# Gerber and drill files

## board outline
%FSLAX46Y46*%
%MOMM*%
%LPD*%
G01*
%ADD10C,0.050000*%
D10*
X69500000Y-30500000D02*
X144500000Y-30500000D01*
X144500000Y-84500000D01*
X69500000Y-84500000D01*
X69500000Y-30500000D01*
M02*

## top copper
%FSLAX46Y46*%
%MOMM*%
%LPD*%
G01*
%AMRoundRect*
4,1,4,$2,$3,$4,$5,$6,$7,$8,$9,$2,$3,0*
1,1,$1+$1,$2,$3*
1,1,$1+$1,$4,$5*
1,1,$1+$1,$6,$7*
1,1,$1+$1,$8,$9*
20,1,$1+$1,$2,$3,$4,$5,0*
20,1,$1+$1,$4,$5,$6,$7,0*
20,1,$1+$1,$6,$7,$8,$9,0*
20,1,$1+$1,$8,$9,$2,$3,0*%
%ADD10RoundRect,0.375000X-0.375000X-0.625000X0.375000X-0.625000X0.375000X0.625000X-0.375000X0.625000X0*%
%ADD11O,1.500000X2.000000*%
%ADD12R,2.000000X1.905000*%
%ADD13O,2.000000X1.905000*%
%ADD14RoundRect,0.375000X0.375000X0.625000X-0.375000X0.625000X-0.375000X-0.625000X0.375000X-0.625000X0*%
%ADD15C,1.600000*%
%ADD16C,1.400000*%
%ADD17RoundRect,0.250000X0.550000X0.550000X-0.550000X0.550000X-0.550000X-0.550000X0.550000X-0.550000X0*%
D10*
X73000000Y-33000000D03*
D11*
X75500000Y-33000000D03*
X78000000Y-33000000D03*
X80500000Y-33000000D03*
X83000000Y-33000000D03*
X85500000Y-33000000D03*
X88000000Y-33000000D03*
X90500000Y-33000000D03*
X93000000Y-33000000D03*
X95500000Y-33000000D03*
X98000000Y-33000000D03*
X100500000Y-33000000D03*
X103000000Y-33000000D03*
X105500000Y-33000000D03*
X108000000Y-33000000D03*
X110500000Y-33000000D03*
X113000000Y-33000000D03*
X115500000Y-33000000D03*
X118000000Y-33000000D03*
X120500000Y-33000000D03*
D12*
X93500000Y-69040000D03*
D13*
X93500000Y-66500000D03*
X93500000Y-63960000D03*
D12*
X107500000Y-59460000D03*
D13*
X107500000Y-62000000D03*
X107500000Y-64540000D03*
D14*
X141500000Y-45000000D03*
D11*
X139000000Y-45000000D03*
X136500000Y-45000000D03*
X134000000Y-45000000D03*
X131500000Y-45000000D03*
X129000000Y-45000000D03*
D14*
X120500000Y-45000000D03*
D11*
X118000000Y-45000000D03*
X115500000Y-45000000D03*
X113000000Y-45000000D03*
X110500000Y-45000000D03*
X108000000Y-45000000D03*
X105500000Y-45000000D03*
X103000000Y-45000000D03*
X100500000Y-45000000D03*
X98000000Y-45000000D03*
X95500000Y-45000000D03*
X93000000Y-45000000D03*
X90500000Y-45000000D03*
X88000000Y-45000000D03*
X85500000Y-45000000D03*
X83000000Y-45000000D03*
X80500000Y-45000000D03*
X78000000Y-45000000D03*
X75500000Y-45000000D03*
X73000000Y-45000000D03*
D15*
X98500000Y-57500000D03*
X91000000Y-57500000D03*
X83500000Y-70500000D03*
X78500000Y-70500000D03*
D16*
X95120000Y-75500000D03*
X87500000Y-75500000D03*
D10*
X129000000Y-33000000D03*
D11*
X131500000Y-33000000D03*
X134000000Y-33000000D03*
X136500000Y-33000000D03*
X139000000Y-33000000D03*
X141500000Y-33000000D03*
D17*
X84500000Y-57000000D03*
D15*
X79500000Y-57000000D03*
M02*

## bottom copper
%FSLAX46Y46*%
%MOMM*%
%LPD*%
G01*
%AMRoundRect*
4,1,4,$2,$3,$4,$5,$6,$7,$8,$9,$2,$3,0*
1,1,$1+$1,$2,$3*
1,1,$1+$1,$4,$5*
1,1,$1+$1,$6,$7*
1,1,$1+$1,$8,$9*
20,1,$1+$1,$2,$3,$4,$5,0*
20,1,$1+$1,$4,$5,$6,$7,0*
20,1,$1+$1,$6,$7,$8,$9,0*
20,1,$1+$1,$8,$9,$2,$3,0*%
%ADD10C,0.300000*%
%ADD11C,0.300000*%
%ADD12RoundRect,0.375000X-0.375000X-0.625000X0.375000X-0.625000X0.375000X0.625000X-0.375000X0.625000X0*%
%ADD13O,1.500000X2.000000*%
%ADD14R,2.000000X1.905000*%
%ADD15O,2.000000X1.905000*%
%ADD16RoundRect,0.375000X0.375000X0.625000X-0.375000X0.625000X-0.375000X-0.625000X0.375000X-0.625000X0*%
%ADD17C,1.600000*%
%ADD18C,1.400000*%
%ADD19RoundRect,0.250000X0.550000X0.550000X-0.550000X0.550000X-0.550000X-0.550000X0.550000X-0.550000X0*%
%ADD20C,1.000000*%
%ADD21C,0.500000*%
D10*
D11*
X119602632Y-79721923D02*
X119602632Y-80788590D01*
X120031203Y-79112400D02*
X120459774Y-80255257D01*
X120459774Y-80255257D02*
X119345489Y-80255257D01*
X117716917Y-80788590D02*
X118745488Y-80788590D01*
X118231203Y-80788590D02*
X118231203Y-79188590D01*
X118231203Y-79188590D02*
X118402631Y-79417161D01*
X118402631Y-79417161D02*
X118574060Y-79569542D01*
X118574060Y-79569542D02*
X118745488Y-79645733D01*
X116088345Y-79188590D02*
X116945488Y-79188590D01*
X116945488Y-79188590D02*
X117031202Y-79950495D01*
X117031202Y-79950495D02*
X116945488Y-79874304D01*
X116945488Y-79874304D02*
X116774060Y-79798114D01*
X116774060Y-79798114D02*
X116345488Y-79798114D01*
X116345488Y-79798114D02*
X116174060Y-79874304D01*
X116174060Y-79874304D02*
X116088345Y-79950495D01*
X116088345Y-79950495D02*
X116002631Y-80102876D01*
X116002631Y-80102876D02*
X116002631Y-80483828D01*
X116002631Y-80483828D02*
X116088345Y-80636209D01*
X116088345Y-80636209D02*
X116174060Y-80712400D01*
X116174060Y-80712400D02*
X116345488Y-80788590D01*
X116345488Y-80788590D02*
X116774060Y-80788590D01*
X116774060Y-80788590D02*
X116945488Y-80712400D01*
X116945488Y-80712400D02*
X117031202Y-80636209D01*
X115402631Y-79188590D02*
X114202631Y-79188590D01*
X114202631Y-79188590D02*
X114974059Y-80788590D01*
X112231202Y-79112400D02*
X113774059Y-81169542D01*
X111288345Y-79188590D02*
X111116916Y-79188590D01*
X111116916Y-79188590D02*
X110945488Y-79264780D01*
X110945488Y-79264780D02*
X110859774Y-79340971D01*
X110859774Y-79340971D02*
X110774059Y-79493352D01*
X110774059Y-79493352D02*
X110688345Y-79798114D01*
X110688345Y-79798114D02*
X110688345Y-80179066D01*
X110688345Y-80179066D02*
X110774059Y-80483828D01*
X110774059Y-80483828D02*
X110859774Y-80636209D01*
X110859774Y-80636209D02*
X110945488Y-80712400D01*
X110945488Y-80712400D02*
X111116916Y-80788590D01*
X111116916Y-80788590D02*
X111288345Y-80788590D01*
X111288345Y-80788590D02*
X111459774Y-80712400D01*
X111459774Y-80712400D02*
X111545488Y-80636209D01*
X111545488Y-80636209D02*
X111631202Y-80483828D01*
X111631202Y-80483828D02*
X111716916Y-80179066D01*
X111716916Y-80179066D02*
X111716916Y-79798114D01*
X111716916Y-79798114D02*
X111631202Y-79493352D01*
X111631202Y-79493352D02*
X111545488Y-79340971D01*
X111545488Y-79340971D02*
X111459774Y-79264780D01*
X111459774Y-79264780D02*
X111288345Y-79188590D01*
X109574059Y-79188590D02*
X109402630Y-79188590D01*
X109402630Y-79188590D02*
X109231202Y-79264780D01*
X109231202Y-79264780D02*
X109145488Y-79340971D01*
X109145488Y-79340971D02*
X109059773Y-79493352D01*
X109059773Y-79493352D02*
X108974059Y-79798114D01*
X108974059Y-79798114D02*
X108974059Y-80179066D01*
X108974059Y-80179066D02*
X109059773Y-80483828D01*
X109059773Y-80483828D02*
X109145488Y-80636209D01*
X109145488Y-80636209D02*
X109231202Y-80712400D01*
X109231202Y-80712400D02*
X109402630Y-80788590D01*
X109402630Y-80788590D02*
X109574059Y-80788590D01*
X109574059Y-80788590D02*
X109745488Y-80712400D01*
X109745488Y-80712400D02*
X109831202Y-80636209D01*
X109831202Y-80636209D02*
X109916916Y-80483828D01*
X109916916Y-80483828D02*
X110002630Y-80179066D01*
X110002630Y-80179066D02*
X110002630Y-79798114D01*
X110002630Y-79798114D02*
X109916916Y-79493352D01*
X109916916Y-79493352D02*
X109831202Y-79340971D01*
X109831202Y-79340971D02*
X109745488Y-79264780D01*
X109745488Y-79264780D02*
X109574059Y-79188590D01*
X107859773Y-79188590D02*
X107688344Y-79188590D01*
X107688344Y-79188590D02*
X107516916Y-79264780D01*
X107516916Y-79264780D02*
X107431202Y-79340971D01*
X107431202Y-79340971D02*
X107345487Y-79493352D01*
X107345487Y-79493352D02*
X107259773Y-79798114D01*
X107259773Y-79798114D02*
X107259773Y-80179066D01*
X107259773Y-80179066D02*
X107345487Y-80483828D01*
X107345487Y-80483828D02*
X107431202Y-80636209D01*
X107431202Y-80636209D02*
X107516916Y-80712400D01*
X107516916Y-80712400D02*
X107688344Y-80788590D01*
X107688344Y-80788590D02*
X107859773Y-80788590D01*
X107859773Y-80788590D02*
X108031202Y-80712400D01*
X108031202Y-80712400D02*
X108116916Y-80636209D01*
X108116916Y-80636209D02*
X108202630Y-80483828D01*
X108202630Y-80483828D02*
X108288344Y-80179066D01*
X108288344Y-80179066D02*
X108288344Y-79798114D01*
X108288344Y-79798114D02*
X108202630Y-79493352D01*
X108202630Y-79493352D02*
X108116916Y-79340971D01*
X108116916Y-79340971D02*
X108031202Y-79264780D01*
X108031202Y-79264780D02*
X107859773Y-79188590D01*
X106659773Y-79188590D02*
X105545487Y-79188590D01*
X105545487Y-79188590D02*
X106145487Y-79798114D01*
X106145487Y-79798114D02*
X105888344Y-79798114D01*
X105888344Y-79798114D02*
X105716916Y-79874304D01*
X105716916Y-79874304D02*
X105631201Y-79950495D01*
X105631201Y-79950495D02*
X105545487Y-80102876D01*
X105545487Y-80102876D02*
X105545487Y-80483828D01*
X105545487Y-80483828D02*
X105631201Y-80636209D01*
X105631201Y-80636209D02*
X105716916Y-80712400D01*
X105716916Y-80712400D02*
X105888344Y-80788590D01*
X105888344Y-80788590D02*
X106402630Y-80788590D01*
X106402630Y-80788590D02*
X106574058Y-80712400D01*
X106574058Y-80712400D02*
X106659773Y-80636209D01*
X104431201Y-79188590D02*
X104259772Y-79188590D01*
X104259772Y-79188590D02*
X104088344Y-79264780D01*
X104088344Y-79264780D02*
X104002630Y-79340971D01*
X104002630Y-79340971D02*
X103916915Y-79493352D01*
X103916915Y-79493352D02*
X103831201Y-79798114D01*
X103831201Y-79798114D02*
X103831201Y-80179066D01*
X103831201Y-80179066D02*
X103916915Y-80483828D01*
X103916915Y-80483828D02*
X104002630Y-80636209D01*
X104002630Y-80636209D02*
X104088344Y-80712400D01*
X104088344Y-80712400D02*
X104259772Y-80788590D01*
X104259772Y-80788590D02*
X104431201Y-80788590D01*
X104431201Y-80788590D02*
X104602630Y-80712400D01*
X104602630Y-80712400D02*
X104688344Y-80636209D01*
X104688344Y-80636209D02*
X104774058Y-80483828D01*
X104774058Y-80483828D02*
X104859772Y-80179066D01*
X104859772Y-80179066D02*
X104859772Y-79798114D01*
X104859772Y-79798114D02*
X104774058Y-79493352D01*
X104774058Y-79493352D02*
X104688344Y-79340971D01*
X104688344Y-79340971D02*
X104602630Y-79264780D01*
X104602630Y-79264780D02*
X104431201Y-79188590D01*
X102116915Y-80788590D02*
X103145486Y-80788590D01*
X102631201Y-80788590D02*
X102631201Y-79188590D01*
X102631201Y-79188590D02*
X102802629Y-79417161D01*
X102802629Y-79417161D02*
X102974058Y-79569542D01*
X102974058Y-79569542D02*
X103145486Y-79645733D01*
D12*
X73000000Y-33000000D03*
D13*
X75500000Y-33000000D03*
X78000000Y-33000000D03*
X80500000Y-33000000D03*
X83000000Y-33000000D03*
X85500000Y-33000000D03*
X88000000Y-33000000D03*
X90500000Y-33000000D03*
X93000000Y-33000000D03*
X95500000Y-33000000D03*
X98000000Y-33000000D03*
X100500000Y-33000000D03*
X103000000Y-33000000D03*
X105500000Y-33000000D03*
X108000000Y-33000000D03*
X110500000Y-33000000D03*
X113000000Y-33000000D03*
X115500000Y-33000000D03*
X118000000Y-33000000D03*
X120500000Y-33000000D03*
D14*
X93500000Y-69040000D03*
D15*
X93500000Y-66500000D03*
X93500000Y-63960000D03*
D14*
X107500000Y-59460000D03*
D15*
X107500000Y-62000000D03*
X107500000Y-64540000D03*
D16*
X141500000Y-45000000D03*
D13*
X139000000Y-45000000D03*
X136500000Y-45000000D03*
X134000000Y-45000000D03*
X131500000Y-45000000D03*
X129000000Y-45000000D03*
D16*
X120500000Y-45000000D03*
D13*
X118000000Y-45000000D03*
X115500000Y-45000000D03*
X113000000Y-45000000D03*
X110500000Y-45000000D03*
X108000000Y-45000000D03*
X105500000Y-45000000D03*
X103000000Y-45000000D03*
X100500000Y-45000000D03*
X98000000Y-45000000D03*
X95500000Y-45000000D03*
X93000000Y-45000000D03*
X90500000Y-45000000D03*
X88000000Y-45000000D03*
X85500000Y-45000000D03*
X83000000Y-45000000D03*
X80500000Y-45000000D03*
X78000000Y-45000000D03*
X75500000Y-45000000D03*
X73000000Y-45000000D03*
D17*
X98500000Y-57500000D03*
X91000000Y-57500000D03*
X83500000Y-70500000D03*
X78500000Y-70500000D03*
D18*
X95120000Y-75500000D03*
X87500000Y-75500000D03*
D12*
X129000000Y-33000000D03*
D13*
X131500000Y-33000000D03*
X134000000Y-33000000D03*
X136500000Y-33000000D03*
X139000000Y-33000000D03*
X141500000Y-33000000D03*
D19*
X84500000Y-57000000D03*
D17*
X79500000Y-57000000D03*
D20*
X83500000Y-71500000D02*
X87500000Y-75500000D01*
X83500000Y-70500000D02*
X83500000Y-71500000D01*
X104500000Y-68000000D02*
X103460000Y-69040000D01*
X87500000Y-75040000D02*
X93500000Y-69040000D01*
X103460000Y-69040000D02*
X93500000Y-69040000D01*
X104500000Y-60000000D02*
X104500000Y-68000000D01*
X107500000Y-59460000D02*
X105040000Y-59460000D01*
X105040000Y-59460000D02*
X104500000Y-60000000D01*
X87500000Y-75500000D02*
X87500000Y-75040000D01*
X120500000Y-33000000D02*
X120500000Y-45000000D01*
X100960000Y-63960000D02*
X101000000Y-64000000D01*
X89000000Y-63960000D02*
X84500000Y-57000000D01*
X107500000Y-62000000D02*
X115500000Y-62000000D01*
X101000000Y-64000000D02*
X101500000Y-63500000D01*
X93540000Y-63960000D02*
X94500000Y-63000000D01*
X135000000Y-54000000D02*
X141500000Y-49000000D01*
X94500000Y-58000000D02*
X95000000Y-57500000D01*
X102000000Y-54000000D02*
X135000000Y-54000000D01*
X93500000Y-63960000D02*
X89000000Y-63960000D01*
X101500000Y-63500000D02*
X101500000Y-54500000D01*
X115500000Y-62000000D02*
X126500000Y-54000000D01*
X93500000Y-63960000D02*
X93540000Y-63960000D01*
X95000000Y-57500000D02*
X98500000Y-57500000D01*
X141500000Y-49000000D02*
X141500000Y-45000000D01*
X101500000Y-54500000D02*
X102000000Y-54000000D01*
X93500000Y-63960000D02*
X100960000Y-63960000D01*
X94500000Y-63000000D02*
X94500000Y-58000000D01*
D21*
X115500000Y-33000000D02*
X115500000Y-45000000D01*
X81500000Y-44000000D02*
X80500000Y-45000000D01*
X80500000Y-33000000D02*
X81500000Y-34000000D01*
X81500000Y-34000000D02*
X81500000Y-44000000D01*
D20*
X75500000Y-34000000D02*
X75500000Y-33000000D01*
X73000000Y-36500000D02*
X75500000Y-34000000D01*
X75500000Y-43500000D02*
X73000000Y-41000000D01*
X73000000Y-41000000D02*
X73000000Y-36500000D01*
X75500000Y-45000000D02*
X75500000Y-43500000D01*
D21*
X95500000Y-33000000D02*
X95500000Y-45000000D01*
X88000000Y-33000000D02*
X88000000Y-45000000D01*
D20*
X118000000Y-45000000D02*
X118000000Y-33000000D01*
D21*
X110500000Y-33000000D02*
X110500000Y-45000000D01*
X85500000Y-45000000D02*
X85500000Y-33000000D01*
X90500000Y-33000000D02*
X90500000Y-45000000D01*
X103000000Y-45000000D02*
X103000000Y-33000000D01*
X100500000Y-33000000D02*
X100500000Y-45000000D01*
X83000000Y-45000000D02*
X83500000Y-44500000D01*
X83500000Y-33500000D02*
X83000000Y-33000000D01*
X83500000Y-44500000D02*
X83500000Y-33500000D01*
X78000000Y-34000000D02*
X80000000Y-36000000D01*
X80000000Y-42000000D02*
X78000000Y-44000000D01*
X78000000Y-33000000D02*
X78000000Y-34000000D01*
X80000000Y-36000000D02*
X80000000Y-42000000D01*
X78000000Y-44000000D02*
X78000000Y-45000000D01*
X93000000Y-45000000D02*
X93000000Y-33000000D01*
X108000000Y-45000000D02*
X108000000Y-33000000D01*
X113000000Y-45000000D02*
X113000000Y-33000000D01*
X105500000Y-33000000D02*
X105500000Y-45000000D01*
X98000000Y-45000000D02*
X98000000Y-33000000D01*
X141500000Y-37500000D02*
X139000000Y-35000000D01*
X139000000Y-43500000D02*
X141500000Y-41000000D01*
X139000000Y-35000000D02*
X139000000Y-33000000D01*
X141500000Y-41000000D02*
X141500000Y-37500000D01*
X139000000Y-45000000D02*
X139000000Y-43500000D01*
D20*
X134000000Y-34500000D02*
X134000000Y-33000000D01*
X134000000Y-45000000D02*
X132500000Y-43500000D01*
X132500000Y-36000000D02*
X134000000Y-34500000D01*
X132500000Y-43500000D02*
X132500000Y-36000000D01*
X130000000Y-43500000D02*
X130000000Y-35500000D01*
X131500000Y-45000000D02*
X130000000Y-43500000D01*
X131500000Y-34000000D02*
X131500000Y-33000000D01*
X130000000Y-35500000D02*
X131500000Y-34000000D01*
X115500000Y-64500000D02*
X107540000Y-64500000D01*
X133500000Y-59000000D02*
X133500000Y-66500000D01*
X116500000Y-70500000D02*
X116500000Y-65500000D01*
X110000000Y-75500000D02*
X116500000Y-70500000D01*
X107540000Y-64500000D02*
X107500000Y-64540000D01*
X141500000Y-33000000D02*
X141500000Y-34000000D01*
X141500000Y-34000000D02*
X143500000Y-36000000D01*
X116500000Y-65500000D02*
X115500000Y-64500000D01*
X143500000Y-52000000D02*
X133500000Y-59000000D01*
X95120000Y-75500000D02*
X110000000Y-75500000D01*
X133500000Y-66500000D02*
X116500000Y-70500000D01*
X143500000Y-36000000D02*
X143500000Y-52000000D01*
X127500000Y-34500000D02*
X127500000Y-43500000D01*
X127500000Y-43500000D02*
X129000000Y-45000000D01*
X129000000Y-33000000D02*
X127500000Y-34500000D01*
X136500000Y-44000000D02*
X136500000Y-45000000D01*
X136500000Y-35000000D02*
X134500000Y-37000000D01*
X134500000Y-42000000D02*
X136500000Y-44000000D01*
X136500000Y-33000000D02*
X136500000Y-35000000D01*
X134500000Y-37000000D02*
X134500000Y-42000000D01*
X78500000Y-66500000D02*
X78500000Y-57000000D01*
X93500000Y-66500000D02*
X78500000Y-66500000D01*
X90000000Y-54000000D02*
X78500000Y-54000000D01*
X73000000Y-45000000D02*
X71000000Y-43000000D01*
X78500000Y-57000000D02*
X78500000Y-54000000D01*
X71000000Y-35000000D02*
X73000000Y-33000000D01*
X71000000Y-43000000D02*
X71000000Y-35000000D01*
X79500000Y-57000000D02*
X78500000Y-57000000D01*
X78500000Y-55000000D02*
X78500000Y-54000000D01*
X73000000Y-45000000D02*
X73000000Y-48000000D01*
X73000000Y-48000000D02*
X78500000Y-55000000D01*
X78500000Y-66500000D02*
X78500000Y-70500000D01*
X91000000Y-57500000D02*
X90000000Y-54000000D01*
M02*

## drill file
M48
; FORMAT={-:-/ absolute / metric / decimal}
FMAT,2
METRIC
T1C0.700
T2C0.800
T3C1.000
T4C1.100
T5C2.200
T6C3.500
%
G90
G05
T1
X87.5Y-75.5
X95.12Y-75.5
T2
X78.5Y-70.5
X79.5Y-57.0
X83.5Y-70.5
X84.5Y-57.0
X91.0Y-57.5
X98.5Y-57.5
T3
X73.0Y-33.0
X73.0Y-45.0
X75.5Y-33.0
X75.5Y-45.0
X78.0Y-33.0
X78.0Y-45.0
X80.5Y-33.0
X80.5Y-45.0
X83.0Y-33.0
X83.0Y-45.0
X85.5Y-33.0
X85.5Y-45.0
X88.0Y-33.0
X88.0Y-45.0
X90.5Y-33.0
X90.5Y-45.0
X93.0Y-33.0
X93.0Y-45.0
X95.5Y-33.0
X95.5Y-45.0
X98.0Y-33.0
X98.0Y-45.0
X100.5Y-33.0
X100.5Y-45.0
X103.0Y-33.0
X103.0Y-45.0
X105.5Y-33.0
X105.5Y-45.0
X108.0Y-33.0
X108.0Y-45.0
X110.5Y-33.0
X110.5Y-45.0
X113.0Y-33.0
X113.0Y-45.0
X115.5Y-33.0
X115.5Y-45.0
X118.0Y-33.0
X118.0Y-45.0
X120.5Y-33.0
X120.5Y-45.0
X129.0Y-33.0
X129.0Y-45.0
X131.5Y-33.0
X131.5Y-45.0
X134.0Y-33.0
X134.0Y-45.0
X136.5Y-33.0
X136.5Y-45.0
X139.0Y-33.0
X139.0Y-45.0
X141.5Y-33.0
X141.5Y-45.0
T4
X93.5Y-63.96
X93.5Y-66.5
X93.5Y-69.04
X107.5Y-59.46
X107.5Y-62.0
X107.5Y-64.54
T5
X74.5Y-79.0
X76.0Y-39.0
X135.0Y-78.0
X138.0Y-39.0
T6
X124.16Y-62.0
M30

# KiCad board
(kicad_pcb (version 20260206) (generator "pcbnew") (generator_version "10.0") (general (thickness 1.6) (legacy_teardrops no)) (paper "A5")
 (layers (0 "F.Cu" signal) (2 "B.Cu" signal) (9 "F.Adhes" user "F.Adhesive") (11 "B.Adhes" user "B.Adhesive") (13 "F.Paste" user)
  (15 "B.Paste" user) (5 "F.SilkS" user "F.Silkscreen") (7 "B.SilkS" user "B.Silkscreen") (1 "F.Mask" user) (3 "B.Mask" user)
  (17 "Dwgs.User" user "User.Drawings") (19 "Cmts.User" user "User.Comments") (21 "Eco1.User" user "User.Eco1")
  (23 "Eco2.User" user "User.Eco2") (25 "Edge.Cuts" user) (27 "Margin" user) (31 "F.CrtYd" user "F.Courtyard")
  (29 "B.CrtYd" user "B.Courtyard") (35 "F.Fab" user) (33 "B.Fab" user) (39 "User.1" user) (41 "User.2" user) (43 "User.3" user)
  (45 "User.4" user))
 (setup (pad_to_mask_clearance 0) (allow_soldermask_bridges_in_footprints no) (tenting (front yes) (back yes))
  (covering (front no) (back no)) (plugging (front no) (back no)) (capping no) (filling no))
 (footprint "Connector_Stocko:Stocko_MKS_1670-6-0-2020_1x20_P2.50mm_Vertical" (layer "F.Cu") (at 73 33)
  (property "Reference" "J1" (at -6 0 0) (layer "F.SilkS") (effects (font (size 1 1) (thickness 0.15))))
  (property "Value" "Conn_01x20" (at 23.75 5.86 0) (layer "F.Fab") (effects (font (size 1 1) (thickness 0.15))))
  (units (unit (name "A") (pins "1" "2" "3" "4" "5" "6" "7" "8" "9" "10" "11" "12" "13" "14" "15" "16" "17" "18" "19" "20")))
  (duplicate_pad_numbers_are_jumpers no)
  (pad "1" thru_hole roundrect (at 0 0) (size 1.5 2) (drill 1) (layers "*.Cu" "*.Mask") (remove_unused_layers no) (roundrect_rratio 0.25)
   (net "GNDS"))
  (pad "2" thru_hole oval (at 2.5 0) (size 1.5 2) (drill 1) (layers "*.Cu" "*.Mask") (remove_unused_layers no) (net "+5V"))
  (pad "3" thru_hole oval (at 5 0) (size 1.5 2) (drill 1) (layers "*.Cu" "*.Mask") (remove_unused_layers no) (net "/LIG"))
  (pad "4" thru_hole oval (at 7.5 0) (size 1.5 2) (drill 1) (layers "*.Cu" "*.Mask") (remove_unused_layers no) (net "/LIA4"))
  (pad "5" thru_hole oval (at 10 0) (size 1.5 2) (drill 1) (layers "*.Cu" "*.Mask") (remove_unused_layers no) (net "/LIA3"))
  (pad "6" thru_hole oval (at 12.5 0) (size 1.5 2) (drill 1) (layers "*.Cu" "*.Mask") (remove_unused_layers no) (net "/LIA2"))
  (pad "7" thru_hole oval (at 15 0) (size 1.5 2) (drill 1) (layers "*.Cu" "*.Mask") (remove_unused_layers no) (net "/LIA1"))
  (pad "8" thru_hole oval (at 17.5 0) (size 1.5 2) (drill 1) (layers "*.Cu" "*.Mask") (remove_unused_layers no) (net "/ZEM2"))
  (pad "9" thru_hole oval (at 20 0) (size 1.5 2) (drill 1) (layers "*.Cu" "*.Mask") (remove_unused_layers no) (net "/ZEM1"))
  (pad "10" thru_hole oval (at 22.5 0) (size 1.5 2) (drill 1) (layers "*.Cu" "*.Mask") (remove_unused_layers no) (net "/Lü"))
  (pad "11" thru_hole oval (at 25 0) (size 1.5 2) (drill 1) (layers "*.Cu" "*.Mask") (remove_unused_layers no) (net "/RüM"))
  (pad "12" thru_hole oval (at 27.5 0) (size 1.5 2) (drill 1) (layers "*.Cu" "*.Mask") (remove_unused_layers no) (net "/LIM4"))
  (pad "13" thru_hole oval (at 30 0) (size 1.5 2) (drill 1) (layers "*.Cu" "*.Mask") (remove_unused_layers no) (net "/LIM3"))
  (pad "14" thru_hole oval (at 32.5 0) (size 1.5 2) (drill 1) (layers "*.Cu" "*.Mask") (remove_unused_layers no) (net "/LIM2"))
  (pad "15" thru_hole oval (at 35 0) (size 1.5 2) (drill 1) (layers "*.Cu" "*.Mask") (remove_unused_layers no) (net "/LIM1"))
  (pad "16" thru_hole oval (at 37.5 0) (size 1.5 2) (drill 1) (layers "*.Cu" "*.Mask") (remove_unused_layers no) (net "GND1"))
  (pad "17" thru_hole oval (at 40 0) (size 1.5 2) (drill 1) (layers "*.Cu" "*.Mask") (remove_unused_layers no) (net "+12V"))
  (pad "18" thru_hole oval (at 42.5 0) (size 1.5 2) (drill 1) (layers "*.Cu" "*.Mask") (remove_unused_layers no) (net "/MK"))
  (pad "19" thru_hole oval (at 45 0) (size 1.5 2) (drill 1) (layers "*.Cu" "*.Mask") (remove_unused_layers no) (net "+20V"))
  (pad "20" thru_hole oval (at 47.5 0) (size 1.5 2) (drill 1) (layers "*.Cu" "*.Mask") (remove_unused_layers no) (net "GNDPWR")))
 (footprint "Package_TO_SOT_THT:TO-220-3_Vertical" (layer "F.Cu") (at 93.5 69.04 90)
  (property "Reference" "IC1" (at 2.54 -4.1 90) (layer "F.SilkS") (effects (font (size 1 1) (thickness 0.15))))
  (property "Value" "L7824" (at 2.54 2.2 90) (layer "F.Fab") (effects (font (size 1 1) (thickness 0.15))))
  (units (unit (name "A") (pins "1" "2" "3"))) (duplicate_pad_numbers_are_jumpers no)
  (pad "1" thru_hole rect (at 0 0 90) (size 1.905 2) (drill 1.1) (layers "*.Cu" "*.Mask") (remove_unused_layers no) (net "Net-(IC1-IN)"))
  (pad "2" thru_hole oval (at 2.54 0 90) (size 1.905 2) (drill 1.1) (layers "*.Cu" "*.Mask") (remove_unused_layers no) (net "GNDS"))
  (pad "3" thru_hole oval (at 5.08 0 90) (size 1.905 2) (drill 1.1) (layers "*.Cu" "*.Mask") (remove_unused_layers no) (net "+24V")))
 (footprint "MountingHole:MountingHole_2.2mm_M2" (layer "F.Cu") (at 74.5 79)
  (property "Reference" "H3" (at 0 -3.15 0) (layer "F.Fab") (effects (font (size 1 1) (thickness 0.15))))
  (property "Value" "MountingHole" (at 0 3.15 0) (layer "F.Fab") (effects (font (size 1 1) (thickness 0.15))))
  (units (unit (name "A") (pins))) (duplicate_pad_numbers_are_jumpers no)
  (pad "" np_thru_hole circle (at 0 0) (size 2.2 2.2) (drill 2.2) (layers "*.Cu" "*.Mask")))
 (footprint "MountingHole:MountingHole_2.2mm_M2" (layer "F.Cu") (at 135 78)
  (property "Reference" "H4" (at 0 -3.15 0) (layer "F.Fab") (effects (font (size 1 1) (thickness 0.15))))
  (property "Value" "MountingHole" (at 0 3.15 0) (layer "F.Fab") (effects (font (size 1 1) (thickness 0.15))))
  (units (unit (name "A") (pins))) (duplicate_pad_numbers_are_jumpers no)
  (pad "" np_thru_hole circle (at 0 0) (size 2.2 2.2) (drill 2.2) (layers "*.Cu" "*.Mask")))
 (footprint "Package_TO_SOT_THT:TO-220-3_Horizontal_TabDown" (layer "F.Cu") (at 107.5 59.46 -90)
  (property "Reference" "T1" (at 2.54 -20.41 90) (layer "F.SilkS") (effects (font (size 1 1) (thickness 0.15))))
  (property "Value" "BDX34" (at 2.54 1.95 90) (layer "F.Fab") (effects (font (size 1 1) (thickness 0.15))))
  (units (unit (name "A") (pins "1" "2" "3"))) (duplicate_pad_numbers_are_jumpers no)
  (pad "" np_thru_hole circle (at 2.54 -16.66 270) (size 3.5 3.5) (drill 3.5) (layers "*.Cu" "*.Mask"))
  (pad "1" thru_hole rect (at 0 0 270) (size 1.905 2) (drill 1.1) (layers "*.Cu" "*.Mask") (remove_unused_layers no) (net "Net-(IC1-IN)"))
  (pad "2" thru_hole oval (at 2.54 0 270) (size 1.905 2) (drill 1.1) (layers "*.Cu" "*.Mask") (remove_unused_layers no) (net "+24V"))
  (pad "3" thru_hole oval (at 5.08 0 270) (size 1.905 2) (drill 1.1) (layers "*.Cu" "*.Mask") (remove_unused_layers no) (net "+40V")))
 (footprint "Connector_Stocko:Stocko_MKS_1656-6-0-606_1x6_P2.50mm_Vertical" (layer "F.Cu") (at 141.5 45 180)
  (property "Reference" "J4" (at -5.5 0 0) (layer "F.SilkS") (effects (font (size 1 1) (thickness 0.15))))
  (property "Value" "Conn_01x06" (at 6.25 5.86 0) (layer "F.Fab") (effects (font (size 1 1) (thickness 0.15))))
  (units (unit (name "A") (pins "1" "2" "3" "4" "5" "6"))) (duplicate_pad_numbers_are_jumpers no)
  (pad "1" thru_hole roundrect (at 0 0 180) (size 1.5 2) (drill 1) (layers "*.Cu" "*.Mask") (remove_unused_layers no)
   (roundrect_rratio 0.25) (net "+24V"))
  (pad "2" thru_hole oval (at 2.5 0 180) (size 1.5 2) (drill 1) (layers "*.Cu" "*.Mask") (remove_unused_layers no) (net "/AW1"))
  (pad "3" thru_hole oval (at 5 0 180) (size 1.5 2) (drill 1) (layers "*.Cu" "*.Mask") (remove_unused_layers no) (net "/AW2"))
  (pad "4" thru_hole oval (at 7.5 0 180) (size 1.5 2) (drill 1) (layers "*.Cu" "*.Mask") (remove_unused_layers no) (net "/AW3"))
  (pad "5" thru_hole oval (at 10 0 180) (size 1.5 2) (drill 1) (layers "*.Cu" "*.Mask") (remove_unused_layers no) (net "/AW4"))
  (pad "6" thru_hole oval (at 12.5 0 180) (size 1.5 2) (drill 1) (layers "*.Cu" "*.Mask") (remove_unused_layers no) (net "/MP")))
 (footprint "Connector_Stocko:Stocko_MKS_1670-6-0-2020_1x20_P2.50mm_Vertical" (layer "F.Cu") (at 120.5 45 180)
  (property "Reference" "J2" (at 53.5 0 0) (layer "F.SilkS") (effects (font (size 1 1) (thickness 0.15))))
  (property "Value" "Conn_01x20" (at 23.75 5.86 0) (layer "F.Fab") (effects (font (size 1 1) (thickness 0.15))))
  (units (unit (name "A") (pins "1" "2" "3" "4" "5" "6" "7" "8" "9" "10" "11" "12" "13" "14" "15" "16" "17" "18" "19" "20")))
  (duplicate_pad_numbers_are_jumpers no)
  (pad "1" thru_hole roundrect (at 0 0 180) (size 1.5 2) (drill 1) (layers "*.Cu" "*.Mask") (remove_unused_layers no)
   (roundrect_rratio 0.25) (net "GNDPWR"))
  (pad "2" thru_hole oval (at 2.5 0 180) (size 1.5 2) (drill 1) (layers "*.Cu" "*.Mask") (remove_unused_layers no) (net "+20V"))
  (pad "3" thru_hole oval (at 5 0 180) (size 1.5 2) (drill 1) (layers "*.Cu" "*.Mask") (remove_unused_layers no) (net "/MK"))
  (pad "4" thru_hole oval (at 7.5 0 180) (size 1.5 2) (drill 1) (layers "*.Cu" "*.Mask") (remove_unused_layers no) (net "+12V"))
  (pad "5" thru_hole oval (at 10 0 180) (size 1.5 2) (drill 1) (layers "*.Cu" "*.Mask") (remove_unused_layers no) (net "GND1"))
  (pad "6" thru_hole oval (at 12.5 0 180) (size 1.5 2) (drill 1) (layers "*.Cu" "*.Mask") (remove_unused_layers no) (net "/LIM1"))
  (pad "7" thru_hole oval (at 15 0 180) (size 1.5 2) (drill 1) (layers "*.Cu" "*.Mask") (remove_unused_layers no) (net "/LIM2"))
  (pad "8" thru_hole oval (at 17.5 0 180) (size 1.5 2) (drill 1) (layers "*.Cu" "*.Mask") (remove_unused_layers no) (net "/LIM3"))
  (pad "9" thru_hole oval (at 20 0 180) (size 1.5 2) (drill 1) (layers "*.Cu" "*.Mask") (remove_unused_layers no) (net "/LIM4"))
  (pad "10" thru_hole oval (at 22.5 0 180) (size 1.5 2) (drill 1) (layers "*.Cu" "*.Mask") (remove_unused_layers no) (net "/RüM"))
  (pad "11" thru_hole oval (at 25 0 180) (size 1.5 2) (drill 1) (layers "*.Cu" "*.Mask") (remove_unused_layers no) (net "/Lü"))
  (pad "12" thru_hole oval (at 27.5 0 180) (size 1.5 2) (drill 1) (layers "*.Cu" "*.Mask") (remove_unused_layers no) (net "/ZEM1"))
  (pad "13" thru_hole oval (at 30 0 180) (size 1.5 2) (drill 1) (layers "*.Cu" "*.Mask") (remove_unused_layers no) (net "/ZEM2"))
  (pad "14" thru_hole oval (at 32.5 0 180) (size 1.5 2) (drill 1) (layers "*.Cu" "*.Mask") (remove_unused_layers no) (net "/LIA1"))
  (pad "15" thru_hole oval (at 35 0 180) (size 1.5 2) (drill 1) (layers "*.Cu" "*.Mask") (remove_unused_layers no) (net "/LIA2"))
  (pad "16" thru_hole oval (at 37.5 0 180) (size 1.5 2) (drill 1) (layers "*.Cu" "*.Mask") (remove_unused_layers no) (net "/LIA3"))
  (pad "17" thru_hole oval (at 40 0 180) (size 1.5 2) (drill 1) (layers "*.Cu" "*.Mask") (remove_unused_layers no) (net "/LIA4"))
  (pad "18" thru_hole oval (at 42.5 0 180) (size 1.5 2) (drill 1) (layers "*.Cu" "*.Mask") (remove_unused_layers no) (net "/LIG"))
  (pad "19" thru_hole oval (at 45 0 180) (size 1.5 2) (drill 1) (layers "*.Cu" "*.Mask") (remove_unused_layers no) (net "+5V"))
  (pad "20" thru_hole oval (at 47.5 0 180) (size 1.5 2) (drill 1) (layers "*.Cu" "*.Mask") (remove_unused_layers no) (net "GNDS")))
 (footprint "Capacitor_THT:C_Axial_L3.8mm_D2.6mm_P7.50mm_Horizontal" (layer "F.Cu") (at 98.5 57.5 180)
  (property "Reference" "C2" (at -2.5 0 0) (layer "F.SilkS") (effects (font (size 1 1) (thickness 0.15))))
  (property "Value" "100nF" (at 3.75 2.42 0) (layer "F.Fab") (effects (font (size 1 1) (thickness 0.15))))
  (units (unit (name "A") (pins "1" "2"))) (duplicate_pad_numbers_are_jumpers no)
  (pad "1" thru_hole circle (at 0 0 180) (size 1.6 1.6) (drill 0.8) (layers "*.Cu" "*.Mask") (remove_unused_layers no) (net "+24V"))
  (pad "2" thru_hole circle (at 7.5 0 180) (size 1.6 1.6) (drill 0.8) (layers "*.Cu" "*.Mask") (remove_unused_layers no) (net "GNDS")))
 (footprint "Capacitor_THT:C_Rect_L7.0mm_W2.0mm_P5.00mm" (layer "F.Cu") (at 83.5 70.5 180)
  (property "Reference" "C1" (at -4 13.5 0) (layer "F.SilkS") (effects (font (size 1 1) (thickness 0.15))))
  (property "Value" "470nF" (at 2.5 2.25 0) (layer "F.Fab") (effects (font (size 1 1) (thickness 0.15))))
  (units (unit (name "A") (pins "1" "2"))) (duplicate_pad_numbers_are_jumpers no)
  (pad "1" thru_hole circle (at 0 0 180) (size 1.6 1.6) (drill 0.8) (layers "*.Cu" "*.Mask") (remove_unused_layers no) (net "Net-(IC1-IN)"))
  (pad "2" thru_hole circle (at 5 0 180) (size 1.6 1.6) (drill 0.8) (layers "*.Cu" "*.Mask") (remove_unused_layers no) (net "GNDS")))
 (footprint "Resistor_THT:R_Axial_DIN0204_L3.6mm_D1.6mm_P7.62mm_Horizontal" (layer "F.Cu") (at 95.12 75.5 180)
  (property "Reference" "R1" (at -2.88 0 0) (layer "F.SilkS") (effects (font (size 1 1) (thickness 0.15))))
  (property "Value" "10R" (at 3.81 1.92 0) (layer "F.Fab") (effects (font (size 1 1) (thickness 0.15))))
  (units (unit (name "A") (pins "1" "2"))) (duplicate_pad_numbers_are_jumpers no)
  (pad "1" thru_hole circle (at 0 0 180) (size 1.4 1.4) (drill 0.7) (layers "*.Cu" "*.Mask") (remove_unused_layers no) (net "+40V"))
  (pad "2" thru_hole circle (at 7.62 0 180) (size 1.4 1.4) (drill 0.7) (layers "*.Cu" "*.Mask") (remove_unused_layers no)
   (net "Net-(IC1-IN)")))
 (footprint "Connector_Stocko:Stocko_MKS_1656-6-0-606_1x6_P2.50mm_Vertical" (layer "F.Cu") (at 129 33)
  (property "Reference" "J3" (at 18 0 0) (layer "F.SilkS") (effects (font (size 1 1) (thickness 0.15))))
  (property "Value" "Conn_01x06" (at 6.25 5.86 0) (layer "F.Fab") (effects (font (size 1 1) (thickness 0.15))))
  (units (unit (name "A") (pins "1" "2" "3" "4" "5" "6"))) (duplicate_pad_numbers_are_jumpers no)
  (pad "1" thru_hole roundrect (at 0 0) (size 1.5 2) (drill 1) (layers "*.Cu" "*.Mask") (remove_unused_layers no) (roundrect_rratio 0.25)
   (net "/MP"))
  (pad "2" thru_hole oval (at 2.5 0) (size 1.5 2) (drill 1) (layers "*.Cu" "*.Mask") (remove_unused_layers no) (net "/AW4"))
  (pad "3" thru_hole oval (at 5 0) (size 1.5 2) (drill 1) (layers "*.Cu" "*.Mask") (remove_unused_layers no) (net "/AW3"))
  (pad "4" thru_hole oval (at 7.5 0) (size 1.5 2) (drill 1) (layers "*.Cu" "*.Mask") (remove_unused_layers no) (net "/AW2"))
  (pad "5" thru_hole oval (at 10 0) (size 1.5 2) (drill 1) (layers "*.Cu" "*.Mask") (remove_unused_layers no) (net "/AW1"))
  (pad "6" thru_hole oval (at 12.5 0) (size 1.5 2) (drill 1) (layers "*.Cu" "*.Mask") (remove_unused_layers no) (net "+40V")))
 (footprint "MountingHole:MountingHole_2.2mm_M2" (layer "F.Cu") (at 76 39)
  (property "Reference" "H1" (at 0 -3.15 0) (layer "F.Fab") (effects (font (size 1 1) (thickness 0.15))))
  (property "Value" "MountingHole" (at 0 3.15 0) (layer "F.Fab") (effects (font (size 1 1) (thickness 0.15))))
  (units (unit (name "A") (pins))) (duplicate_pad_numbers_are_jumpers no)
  (pad "" np_thru_hole circle (at 0 0) (size 2.2 2.2) (drill 2.2) (layers "*.Cu" "*.Mask")))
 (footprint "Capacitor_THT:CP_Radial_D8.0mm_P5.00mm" (layer "F.Cu") (at 84.5 57 180)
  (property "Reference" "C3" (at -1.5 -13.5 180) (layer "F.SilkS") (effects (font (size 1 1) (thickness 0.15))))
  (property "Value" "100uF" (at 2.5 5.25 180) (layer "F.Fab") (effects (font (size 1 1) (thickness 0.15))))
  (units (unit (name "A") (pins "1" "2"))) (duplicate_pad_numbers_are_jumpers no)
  (pad "1" thru_hole roundrect (at 0 0 180) (size 1.6 1.6) (drill 0.8) (layers "*.Cu" "*.Mask") (remove_unused_layers no)
   (roundrect_rratio 0.15625) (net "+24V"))
  (pad "2" thru_hole circle (at 5 0 180) (size 1.6 1.6) (drill 0.8) (layers "*.Cu" "*.Mask") (remove_unused_layers no) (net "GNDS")))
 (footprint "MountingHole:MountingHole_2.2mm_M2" (layer "F.Cu") (at 138 39)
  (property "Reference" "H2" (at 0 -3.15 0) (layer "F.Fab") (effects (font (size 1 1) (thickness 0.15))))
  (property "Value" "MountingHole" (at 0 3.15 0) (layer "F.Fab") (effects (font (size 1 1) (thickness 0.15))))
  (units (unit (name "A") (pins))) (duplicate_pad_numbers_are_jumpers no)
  (pad "" np_thru_hole circle (at 0 0) (size 2.2 2.2) (drill 2.2) (layers "*.Cu" "*.Mask")))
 (gr_rect (start 69.5 30.5) (end 144.5 84.5) (stroke (width 0.05) (type default)) (fill no) (layer "Edge.Cuts"))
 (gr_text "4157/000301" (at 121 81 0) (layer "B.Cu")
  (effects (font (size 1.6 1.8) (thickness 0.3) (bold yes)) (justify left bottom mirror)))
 (segment (start 83.5 71.5) (end 87.5 75.5) (width 1) (layer "B.Cu") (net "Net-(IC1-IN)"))
 (segment (start 83.5 70.5) (end 83.5 71.5) (width 1) (layer "B.Cu") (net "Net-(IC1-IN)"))
 (segment (start 104.5 68) (end 103.46 69.04) (width 1) (layer "B.Cu") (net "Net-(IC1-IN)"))
 (segment (start 87.5 75.04) (end 93.5 69.04) (width 1) (layer "B.Cu") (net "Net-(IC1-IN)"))
 (segment (start 103.46 69.04) (end 93.5 69.04) (width 1) (layer "B.Cu") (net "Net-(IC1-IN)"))
 (segment (start 104.5 60) (end 104.5 68) (width 1) (layer "B.Cu") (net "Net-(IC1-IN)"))
 (segment (start 107.5 59.46) (end 105.04 59.46) (width 1) (layer "B.Cu") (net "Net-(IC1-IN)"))
 (segment (start 105.04 59.46) (end 104.5 60) (width 1) (layer "B.Cu") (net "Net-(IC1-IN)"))
 (segment (start 87.5 75.5) (end 87.5 75.04) (width 1) (layer "B.Cu") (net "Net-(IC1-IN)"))
 (segment (start 120.5 33) (end 120.5 45) (width 1) (layer "B.Cu") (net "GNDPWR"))
 (segment (start 100.96 63.96) (end 101 64) (width 1) (layer "B.Cu") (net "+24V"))
 (segment (start 89 63.96) (end 84.5 57) (width 1) (layer "B.Cu") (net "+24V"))
 (segment (start 107.5 62) (end 115.5 62) (width 1) (layer "B.Cu") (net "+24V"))
 (segment (start 101 64) (end 101.5 63.5) (width 1) (layer "B.Cu") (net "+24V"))
 (segment (start 93.54 63.96) (end 94.5 63) (width 1) (layer "B.Cu") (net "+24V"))
 (segment (start 135 54) (end 141.5 49) (width 1) (layer "B.Cu") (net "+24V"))
 (segment (start 94.5 58) (end 95 57.5) (width 1) (layer "B.Cu") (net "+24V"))
 (segment (start 102 54) (end 135 54) (width 1) (layer "B.Cu") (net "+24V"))
 (segment (start 93.5 63.96) (end 89 63.96) (width 1) (layer "B.Cu") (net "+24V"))
 (segment (start 101.5 63.5) (end 101.5 54.5) (width 1) (layer "B.Cu") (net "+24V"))
 (segment (start 115.5 62) (end 126.5 54) (width 1) (layer "B.Cu") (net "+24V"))
 (segment (start 93.5 63.96) (end 93.54 63.96) (width 1) (layer "B.Cu") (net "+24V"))
 (segment (start 95 57.5) (end 98.5 57.5) (width 1) (layer "B.Cu") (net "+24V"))
 (segment (start 141.5 49) (end 141.5 45) (width 1) (layer "B.Cu") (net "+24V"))
 (segment (start 101.5 54.5) (end 102 54) (width 1) (layer "B.Cu") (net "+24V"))
 (segment (start 93.5 63.96) (end 100.96 63.96) (width 1) (layer "B.Cu") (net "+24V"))
 (segment (start 94.5 63) (end 94.5 58) (width 1) (layer "B.Cu") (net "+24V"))
 (segment (start 115.5 33) (end 115.5 45) (width 0.5) (layer "B.Cu") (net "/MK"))
 (segment (start 81.5 44) (end 80.5 45) (width 0.5) (layer "B.Cu") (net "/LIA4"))
 (segment (start 80.5 33) (end 81.5 34) (width 0.5) (layer "B.Cu") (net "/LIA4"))
 (segment (start 81.5 34) (end 81.5 44) (width 0.5) (layer "B.Cu") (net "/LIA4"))
 (segment (start 75.5 34) (end 75.5 33) (width 1) (layer "B.Cu") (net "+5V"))
 (segment (start 73 36.5) (end 75.5 34) (width 1) (layer "B.Cu") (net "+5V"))
 (segment (start 75.5 43.5) (end 73 41) (width 1) (layer "B.Cu") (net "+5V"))
 (segment (start 73 41) (end 73 36.5) (width 1) (layer "B.Cu") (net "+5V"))
 (segment (start 75.5 45) (end 75.5 43.5) (width 1) (layer "B.Cu") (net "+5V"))
 (segment (start 95.5 33) (end 95.5 45) (width 0.5) (layer "B.Cu") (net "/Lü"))
 (segment (start 88 33) (end 88 45) (width 0.5) (layer "B.Cu") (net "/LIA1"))
 (segment (start 118 45) (end 118 33) (width 1) (layer "B.Cu") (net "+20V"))
 (segment (start 110.5 33) (end 110.5 45) (width 0.5) (layer "B.Cu") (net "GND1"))
 (segment (start 85.5 45) (end 85.5 33) (width 0.5) (layer "B.Cu") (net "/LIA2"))
 (segment (start 90.5 33) (end 90.5 45) (width 0.5) (layer "B.Cu") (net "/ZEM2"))
 (segment (start 103 45) (end 103 33) (width 0.5) (layer "B.Cu") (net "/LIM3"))
 (segment (start 100.5 33) (end 100.5 45) (width 0.5) (layer "B.Cu") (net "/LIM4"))
 (segment (start 83 45) (end 83.5 44.5) (width 0.5) (layer "B.Cu") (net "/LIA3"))
 (segment (start 83.5 33.5) (end 83 33) (width 0.5) (layer "B.Cu") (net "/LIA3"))
 (segment (start 83.5 44.5) (end 83.5 33.5) (width 0.5) (layer "B.Cu") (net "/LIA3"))
 (segment (start 78 34) (end 80 36) (width 0.5) (layer "B.Cu") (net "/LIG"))
 (segment (start 80 42) (end 78 44) (width 0.5) (layer "B.Cu") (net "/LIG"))
 (segment (start 78 33) (end 78 34) (width 0.5) (layer "B.Cu") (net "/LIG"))
 (segment (start 80 36) (end 80 42) (width 0.5) (layer "B.Cu") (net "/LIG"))
 (segment (start 78 44) (end 78 45) (width 0.5) (layer "B.Cu") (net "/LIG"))
 (segment (start 93 45) (end 93 33) (width 0.5) (layer "B.Cu") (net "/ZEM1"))
 (segment (start 108 45) (end 108 33) (width 0.5) (layer "B.Cu") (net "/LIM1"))
 (segment (start 113 45) (end 113 33) (width 0.5) (layer "B.Cu") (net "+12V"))
 (segment (start 105.5 33) (end 105.5 45) (width 0.5) (layer "B.Cu") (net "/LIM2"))
 (segment (start 98 45) (end 98 33) (width 0.5) (layer "B.Cu") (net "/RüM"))
 (segment (start 141.5 37.5) (end 139 35) (width 0.5) (layer "B.Cu") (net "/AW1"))
 (segment (start 139 43.5) (end 141.5 41) (width 0.5) (layer "B.Cu") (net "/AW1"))
 (segment (start 139 35) (end 139 33) (width 0.5) (layer "B.Cu") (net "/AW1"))
 (segment (start 141.5 41) (end 141.5 37.5) (width 0.5) (layer "B.Cu") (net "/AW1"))
 (segment (start 139 45) (end 139 43.5) (width 0.5) (layer "B.Cu") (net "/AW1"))
 (segment (start 134 34.5) (end 134 33) (width 1) (layer "B.Cu") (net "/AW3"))
 (segment (start 134 45) (end 132.5 43.5) (width 1) (layer "B.Cu") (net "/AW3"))
 (segment (start 132.5 36) (end 134 34.5) (width 1) (layer "B.Cu") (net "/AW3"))
 (segment (start 132.5 43.5) (end 132.5 36) (width 1) (layer "B.Cu") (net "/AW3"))
 (segment (start 130 43.5) (end 130 35.5) (width 1) (layer "B.Cu") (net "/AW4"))
 (segment (start 131.5 45) (end 130 43.5) (width 1) (layer "B.Cu") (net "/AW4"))
 (segment (start 131.5 34) (end 131.5 33) (width 1) (layer "B.Cu") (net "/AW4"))
 (segment (start 130 35.5) (end 131.5 34) (width 1) (layer "B.Cu") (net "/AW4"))
 (segment (start 115.5 64.5) (end 107.54 64.5) (width 1) (layer "B.Cu") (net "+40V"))
 (segment (start 133.5 59) (end 133.5 66.5) (width 1) (layer "B.Cu") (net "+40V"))
 (segment (start 116.5 70.5) (end 116.5 65.5) (width 1) (layer "B.Cu") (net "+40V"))
 (segment (start 110 75.5) (end 116.5 70.5) (width 1) (layer "B.Cu") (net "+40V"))
 (segment (start 107.54 64.5) (end 107.5 64.54) (width 1) (layer "B.Cu") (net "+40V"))
 (segment (start 141.5 33) (end 141.5 34) (width 1) (layer "B.Cu") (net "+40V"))
 (segment (start 141.5 34) (end 143.5 36) (width 1) (layer "B.Cu") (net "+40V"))
 (segment (start 116.5 65.5) (end 115.5 64.5) (width 1) (layer "B.Cu") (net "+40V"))
 (segment (start 143.5 52) (end 133.5 59) (width 1) (layer "B.Cu") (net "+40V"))
 (segment (start 95.12 75.5) (end 110 75.5) (width 1) (layer "B.Cu") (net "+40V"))
 (segment (start 133.5 66.5) (end 116.5 70.5) (width 1) (layer "B.Cu") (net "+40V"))
 (segment (start 143.5 36) (end 143.5 52) (width 1) (layer "B.Cu") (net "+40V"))
 (segment (start 127.5 34.5) (end 127.5 43.5) (width 1) (layer "B.Cu") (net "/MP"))
 (segment (start 127.5 43.5) (end 129 45) (width 1) (layer "B.Cu") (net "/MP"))
 (segment (start 129 33) (end 127.5 34.5) (width 1) (layer "B.Cu") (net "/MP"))
 (segment (start 136.5 44) (end 136.5 45) (width 1) (layer "B.Cu") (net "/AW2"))
 (segment (start 136.5 35) (end 134.5 37) (width 1) (layer "B.Cu") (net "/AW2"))
 (segment (start 134.5 42) (end 136.5 44) (width 1) (layer "B.Cu") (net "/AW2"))
 (segment (start 136.5 33) (end 136.5 35) (width 1) (layer "B.Cu") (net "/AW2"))
 (segment (start 134.5 37) (end 134.5 42) (width 1) (layer "B.Cu") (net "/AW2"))
 (segment (start 78.5 66.5) (end 78.5 57) (width 1) (layer "B.Cu") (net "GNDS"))
 (segment (start 93.5 66.5) (end 78.5 66.5) (width 1) (layer "B.Cu") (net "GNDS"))
 (segment (start 90 54) (end 78.5 54) (width 1) (layer "B.Cu") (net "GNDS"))
 (segment (start 73 45) (end 71 43) (width 1) (layer "B.Cu") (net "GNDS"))
 (segment (start 78.5 57) (end 78.5 54) (width 1) (layer "B.Cu") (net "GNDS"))
 (segment (start 71 35) (end 73 33) (width 1) (layer "B.Cu") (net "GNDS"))
 (segment (start 71 43) (end 71 35) (width 1) (layer "B.Cu") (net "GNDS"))
 (segment (start 79.5 57) (end 78.5 57) (width 1) (layer "B.Cu") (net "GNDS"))
 (segment (start 78.5 55) (end 78.5 54) (width 1) (layer "B.Cu") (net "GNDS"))
 (segment (start 73 45) (end 73 48) (width 1) (layer "B.Cu") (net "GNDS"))
 (segment (start 73 48) (end 78.5 55) (width 1) (layer "B.Cu") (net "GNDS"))
 (segment (start 78.5 66.5) (end 78.5 70.5) (width 1) (layer "B.Cu") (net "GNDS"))
 (segment (start 91 57.5) (end 90 54) (width 1) (layer "B.Cu") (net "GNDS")))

